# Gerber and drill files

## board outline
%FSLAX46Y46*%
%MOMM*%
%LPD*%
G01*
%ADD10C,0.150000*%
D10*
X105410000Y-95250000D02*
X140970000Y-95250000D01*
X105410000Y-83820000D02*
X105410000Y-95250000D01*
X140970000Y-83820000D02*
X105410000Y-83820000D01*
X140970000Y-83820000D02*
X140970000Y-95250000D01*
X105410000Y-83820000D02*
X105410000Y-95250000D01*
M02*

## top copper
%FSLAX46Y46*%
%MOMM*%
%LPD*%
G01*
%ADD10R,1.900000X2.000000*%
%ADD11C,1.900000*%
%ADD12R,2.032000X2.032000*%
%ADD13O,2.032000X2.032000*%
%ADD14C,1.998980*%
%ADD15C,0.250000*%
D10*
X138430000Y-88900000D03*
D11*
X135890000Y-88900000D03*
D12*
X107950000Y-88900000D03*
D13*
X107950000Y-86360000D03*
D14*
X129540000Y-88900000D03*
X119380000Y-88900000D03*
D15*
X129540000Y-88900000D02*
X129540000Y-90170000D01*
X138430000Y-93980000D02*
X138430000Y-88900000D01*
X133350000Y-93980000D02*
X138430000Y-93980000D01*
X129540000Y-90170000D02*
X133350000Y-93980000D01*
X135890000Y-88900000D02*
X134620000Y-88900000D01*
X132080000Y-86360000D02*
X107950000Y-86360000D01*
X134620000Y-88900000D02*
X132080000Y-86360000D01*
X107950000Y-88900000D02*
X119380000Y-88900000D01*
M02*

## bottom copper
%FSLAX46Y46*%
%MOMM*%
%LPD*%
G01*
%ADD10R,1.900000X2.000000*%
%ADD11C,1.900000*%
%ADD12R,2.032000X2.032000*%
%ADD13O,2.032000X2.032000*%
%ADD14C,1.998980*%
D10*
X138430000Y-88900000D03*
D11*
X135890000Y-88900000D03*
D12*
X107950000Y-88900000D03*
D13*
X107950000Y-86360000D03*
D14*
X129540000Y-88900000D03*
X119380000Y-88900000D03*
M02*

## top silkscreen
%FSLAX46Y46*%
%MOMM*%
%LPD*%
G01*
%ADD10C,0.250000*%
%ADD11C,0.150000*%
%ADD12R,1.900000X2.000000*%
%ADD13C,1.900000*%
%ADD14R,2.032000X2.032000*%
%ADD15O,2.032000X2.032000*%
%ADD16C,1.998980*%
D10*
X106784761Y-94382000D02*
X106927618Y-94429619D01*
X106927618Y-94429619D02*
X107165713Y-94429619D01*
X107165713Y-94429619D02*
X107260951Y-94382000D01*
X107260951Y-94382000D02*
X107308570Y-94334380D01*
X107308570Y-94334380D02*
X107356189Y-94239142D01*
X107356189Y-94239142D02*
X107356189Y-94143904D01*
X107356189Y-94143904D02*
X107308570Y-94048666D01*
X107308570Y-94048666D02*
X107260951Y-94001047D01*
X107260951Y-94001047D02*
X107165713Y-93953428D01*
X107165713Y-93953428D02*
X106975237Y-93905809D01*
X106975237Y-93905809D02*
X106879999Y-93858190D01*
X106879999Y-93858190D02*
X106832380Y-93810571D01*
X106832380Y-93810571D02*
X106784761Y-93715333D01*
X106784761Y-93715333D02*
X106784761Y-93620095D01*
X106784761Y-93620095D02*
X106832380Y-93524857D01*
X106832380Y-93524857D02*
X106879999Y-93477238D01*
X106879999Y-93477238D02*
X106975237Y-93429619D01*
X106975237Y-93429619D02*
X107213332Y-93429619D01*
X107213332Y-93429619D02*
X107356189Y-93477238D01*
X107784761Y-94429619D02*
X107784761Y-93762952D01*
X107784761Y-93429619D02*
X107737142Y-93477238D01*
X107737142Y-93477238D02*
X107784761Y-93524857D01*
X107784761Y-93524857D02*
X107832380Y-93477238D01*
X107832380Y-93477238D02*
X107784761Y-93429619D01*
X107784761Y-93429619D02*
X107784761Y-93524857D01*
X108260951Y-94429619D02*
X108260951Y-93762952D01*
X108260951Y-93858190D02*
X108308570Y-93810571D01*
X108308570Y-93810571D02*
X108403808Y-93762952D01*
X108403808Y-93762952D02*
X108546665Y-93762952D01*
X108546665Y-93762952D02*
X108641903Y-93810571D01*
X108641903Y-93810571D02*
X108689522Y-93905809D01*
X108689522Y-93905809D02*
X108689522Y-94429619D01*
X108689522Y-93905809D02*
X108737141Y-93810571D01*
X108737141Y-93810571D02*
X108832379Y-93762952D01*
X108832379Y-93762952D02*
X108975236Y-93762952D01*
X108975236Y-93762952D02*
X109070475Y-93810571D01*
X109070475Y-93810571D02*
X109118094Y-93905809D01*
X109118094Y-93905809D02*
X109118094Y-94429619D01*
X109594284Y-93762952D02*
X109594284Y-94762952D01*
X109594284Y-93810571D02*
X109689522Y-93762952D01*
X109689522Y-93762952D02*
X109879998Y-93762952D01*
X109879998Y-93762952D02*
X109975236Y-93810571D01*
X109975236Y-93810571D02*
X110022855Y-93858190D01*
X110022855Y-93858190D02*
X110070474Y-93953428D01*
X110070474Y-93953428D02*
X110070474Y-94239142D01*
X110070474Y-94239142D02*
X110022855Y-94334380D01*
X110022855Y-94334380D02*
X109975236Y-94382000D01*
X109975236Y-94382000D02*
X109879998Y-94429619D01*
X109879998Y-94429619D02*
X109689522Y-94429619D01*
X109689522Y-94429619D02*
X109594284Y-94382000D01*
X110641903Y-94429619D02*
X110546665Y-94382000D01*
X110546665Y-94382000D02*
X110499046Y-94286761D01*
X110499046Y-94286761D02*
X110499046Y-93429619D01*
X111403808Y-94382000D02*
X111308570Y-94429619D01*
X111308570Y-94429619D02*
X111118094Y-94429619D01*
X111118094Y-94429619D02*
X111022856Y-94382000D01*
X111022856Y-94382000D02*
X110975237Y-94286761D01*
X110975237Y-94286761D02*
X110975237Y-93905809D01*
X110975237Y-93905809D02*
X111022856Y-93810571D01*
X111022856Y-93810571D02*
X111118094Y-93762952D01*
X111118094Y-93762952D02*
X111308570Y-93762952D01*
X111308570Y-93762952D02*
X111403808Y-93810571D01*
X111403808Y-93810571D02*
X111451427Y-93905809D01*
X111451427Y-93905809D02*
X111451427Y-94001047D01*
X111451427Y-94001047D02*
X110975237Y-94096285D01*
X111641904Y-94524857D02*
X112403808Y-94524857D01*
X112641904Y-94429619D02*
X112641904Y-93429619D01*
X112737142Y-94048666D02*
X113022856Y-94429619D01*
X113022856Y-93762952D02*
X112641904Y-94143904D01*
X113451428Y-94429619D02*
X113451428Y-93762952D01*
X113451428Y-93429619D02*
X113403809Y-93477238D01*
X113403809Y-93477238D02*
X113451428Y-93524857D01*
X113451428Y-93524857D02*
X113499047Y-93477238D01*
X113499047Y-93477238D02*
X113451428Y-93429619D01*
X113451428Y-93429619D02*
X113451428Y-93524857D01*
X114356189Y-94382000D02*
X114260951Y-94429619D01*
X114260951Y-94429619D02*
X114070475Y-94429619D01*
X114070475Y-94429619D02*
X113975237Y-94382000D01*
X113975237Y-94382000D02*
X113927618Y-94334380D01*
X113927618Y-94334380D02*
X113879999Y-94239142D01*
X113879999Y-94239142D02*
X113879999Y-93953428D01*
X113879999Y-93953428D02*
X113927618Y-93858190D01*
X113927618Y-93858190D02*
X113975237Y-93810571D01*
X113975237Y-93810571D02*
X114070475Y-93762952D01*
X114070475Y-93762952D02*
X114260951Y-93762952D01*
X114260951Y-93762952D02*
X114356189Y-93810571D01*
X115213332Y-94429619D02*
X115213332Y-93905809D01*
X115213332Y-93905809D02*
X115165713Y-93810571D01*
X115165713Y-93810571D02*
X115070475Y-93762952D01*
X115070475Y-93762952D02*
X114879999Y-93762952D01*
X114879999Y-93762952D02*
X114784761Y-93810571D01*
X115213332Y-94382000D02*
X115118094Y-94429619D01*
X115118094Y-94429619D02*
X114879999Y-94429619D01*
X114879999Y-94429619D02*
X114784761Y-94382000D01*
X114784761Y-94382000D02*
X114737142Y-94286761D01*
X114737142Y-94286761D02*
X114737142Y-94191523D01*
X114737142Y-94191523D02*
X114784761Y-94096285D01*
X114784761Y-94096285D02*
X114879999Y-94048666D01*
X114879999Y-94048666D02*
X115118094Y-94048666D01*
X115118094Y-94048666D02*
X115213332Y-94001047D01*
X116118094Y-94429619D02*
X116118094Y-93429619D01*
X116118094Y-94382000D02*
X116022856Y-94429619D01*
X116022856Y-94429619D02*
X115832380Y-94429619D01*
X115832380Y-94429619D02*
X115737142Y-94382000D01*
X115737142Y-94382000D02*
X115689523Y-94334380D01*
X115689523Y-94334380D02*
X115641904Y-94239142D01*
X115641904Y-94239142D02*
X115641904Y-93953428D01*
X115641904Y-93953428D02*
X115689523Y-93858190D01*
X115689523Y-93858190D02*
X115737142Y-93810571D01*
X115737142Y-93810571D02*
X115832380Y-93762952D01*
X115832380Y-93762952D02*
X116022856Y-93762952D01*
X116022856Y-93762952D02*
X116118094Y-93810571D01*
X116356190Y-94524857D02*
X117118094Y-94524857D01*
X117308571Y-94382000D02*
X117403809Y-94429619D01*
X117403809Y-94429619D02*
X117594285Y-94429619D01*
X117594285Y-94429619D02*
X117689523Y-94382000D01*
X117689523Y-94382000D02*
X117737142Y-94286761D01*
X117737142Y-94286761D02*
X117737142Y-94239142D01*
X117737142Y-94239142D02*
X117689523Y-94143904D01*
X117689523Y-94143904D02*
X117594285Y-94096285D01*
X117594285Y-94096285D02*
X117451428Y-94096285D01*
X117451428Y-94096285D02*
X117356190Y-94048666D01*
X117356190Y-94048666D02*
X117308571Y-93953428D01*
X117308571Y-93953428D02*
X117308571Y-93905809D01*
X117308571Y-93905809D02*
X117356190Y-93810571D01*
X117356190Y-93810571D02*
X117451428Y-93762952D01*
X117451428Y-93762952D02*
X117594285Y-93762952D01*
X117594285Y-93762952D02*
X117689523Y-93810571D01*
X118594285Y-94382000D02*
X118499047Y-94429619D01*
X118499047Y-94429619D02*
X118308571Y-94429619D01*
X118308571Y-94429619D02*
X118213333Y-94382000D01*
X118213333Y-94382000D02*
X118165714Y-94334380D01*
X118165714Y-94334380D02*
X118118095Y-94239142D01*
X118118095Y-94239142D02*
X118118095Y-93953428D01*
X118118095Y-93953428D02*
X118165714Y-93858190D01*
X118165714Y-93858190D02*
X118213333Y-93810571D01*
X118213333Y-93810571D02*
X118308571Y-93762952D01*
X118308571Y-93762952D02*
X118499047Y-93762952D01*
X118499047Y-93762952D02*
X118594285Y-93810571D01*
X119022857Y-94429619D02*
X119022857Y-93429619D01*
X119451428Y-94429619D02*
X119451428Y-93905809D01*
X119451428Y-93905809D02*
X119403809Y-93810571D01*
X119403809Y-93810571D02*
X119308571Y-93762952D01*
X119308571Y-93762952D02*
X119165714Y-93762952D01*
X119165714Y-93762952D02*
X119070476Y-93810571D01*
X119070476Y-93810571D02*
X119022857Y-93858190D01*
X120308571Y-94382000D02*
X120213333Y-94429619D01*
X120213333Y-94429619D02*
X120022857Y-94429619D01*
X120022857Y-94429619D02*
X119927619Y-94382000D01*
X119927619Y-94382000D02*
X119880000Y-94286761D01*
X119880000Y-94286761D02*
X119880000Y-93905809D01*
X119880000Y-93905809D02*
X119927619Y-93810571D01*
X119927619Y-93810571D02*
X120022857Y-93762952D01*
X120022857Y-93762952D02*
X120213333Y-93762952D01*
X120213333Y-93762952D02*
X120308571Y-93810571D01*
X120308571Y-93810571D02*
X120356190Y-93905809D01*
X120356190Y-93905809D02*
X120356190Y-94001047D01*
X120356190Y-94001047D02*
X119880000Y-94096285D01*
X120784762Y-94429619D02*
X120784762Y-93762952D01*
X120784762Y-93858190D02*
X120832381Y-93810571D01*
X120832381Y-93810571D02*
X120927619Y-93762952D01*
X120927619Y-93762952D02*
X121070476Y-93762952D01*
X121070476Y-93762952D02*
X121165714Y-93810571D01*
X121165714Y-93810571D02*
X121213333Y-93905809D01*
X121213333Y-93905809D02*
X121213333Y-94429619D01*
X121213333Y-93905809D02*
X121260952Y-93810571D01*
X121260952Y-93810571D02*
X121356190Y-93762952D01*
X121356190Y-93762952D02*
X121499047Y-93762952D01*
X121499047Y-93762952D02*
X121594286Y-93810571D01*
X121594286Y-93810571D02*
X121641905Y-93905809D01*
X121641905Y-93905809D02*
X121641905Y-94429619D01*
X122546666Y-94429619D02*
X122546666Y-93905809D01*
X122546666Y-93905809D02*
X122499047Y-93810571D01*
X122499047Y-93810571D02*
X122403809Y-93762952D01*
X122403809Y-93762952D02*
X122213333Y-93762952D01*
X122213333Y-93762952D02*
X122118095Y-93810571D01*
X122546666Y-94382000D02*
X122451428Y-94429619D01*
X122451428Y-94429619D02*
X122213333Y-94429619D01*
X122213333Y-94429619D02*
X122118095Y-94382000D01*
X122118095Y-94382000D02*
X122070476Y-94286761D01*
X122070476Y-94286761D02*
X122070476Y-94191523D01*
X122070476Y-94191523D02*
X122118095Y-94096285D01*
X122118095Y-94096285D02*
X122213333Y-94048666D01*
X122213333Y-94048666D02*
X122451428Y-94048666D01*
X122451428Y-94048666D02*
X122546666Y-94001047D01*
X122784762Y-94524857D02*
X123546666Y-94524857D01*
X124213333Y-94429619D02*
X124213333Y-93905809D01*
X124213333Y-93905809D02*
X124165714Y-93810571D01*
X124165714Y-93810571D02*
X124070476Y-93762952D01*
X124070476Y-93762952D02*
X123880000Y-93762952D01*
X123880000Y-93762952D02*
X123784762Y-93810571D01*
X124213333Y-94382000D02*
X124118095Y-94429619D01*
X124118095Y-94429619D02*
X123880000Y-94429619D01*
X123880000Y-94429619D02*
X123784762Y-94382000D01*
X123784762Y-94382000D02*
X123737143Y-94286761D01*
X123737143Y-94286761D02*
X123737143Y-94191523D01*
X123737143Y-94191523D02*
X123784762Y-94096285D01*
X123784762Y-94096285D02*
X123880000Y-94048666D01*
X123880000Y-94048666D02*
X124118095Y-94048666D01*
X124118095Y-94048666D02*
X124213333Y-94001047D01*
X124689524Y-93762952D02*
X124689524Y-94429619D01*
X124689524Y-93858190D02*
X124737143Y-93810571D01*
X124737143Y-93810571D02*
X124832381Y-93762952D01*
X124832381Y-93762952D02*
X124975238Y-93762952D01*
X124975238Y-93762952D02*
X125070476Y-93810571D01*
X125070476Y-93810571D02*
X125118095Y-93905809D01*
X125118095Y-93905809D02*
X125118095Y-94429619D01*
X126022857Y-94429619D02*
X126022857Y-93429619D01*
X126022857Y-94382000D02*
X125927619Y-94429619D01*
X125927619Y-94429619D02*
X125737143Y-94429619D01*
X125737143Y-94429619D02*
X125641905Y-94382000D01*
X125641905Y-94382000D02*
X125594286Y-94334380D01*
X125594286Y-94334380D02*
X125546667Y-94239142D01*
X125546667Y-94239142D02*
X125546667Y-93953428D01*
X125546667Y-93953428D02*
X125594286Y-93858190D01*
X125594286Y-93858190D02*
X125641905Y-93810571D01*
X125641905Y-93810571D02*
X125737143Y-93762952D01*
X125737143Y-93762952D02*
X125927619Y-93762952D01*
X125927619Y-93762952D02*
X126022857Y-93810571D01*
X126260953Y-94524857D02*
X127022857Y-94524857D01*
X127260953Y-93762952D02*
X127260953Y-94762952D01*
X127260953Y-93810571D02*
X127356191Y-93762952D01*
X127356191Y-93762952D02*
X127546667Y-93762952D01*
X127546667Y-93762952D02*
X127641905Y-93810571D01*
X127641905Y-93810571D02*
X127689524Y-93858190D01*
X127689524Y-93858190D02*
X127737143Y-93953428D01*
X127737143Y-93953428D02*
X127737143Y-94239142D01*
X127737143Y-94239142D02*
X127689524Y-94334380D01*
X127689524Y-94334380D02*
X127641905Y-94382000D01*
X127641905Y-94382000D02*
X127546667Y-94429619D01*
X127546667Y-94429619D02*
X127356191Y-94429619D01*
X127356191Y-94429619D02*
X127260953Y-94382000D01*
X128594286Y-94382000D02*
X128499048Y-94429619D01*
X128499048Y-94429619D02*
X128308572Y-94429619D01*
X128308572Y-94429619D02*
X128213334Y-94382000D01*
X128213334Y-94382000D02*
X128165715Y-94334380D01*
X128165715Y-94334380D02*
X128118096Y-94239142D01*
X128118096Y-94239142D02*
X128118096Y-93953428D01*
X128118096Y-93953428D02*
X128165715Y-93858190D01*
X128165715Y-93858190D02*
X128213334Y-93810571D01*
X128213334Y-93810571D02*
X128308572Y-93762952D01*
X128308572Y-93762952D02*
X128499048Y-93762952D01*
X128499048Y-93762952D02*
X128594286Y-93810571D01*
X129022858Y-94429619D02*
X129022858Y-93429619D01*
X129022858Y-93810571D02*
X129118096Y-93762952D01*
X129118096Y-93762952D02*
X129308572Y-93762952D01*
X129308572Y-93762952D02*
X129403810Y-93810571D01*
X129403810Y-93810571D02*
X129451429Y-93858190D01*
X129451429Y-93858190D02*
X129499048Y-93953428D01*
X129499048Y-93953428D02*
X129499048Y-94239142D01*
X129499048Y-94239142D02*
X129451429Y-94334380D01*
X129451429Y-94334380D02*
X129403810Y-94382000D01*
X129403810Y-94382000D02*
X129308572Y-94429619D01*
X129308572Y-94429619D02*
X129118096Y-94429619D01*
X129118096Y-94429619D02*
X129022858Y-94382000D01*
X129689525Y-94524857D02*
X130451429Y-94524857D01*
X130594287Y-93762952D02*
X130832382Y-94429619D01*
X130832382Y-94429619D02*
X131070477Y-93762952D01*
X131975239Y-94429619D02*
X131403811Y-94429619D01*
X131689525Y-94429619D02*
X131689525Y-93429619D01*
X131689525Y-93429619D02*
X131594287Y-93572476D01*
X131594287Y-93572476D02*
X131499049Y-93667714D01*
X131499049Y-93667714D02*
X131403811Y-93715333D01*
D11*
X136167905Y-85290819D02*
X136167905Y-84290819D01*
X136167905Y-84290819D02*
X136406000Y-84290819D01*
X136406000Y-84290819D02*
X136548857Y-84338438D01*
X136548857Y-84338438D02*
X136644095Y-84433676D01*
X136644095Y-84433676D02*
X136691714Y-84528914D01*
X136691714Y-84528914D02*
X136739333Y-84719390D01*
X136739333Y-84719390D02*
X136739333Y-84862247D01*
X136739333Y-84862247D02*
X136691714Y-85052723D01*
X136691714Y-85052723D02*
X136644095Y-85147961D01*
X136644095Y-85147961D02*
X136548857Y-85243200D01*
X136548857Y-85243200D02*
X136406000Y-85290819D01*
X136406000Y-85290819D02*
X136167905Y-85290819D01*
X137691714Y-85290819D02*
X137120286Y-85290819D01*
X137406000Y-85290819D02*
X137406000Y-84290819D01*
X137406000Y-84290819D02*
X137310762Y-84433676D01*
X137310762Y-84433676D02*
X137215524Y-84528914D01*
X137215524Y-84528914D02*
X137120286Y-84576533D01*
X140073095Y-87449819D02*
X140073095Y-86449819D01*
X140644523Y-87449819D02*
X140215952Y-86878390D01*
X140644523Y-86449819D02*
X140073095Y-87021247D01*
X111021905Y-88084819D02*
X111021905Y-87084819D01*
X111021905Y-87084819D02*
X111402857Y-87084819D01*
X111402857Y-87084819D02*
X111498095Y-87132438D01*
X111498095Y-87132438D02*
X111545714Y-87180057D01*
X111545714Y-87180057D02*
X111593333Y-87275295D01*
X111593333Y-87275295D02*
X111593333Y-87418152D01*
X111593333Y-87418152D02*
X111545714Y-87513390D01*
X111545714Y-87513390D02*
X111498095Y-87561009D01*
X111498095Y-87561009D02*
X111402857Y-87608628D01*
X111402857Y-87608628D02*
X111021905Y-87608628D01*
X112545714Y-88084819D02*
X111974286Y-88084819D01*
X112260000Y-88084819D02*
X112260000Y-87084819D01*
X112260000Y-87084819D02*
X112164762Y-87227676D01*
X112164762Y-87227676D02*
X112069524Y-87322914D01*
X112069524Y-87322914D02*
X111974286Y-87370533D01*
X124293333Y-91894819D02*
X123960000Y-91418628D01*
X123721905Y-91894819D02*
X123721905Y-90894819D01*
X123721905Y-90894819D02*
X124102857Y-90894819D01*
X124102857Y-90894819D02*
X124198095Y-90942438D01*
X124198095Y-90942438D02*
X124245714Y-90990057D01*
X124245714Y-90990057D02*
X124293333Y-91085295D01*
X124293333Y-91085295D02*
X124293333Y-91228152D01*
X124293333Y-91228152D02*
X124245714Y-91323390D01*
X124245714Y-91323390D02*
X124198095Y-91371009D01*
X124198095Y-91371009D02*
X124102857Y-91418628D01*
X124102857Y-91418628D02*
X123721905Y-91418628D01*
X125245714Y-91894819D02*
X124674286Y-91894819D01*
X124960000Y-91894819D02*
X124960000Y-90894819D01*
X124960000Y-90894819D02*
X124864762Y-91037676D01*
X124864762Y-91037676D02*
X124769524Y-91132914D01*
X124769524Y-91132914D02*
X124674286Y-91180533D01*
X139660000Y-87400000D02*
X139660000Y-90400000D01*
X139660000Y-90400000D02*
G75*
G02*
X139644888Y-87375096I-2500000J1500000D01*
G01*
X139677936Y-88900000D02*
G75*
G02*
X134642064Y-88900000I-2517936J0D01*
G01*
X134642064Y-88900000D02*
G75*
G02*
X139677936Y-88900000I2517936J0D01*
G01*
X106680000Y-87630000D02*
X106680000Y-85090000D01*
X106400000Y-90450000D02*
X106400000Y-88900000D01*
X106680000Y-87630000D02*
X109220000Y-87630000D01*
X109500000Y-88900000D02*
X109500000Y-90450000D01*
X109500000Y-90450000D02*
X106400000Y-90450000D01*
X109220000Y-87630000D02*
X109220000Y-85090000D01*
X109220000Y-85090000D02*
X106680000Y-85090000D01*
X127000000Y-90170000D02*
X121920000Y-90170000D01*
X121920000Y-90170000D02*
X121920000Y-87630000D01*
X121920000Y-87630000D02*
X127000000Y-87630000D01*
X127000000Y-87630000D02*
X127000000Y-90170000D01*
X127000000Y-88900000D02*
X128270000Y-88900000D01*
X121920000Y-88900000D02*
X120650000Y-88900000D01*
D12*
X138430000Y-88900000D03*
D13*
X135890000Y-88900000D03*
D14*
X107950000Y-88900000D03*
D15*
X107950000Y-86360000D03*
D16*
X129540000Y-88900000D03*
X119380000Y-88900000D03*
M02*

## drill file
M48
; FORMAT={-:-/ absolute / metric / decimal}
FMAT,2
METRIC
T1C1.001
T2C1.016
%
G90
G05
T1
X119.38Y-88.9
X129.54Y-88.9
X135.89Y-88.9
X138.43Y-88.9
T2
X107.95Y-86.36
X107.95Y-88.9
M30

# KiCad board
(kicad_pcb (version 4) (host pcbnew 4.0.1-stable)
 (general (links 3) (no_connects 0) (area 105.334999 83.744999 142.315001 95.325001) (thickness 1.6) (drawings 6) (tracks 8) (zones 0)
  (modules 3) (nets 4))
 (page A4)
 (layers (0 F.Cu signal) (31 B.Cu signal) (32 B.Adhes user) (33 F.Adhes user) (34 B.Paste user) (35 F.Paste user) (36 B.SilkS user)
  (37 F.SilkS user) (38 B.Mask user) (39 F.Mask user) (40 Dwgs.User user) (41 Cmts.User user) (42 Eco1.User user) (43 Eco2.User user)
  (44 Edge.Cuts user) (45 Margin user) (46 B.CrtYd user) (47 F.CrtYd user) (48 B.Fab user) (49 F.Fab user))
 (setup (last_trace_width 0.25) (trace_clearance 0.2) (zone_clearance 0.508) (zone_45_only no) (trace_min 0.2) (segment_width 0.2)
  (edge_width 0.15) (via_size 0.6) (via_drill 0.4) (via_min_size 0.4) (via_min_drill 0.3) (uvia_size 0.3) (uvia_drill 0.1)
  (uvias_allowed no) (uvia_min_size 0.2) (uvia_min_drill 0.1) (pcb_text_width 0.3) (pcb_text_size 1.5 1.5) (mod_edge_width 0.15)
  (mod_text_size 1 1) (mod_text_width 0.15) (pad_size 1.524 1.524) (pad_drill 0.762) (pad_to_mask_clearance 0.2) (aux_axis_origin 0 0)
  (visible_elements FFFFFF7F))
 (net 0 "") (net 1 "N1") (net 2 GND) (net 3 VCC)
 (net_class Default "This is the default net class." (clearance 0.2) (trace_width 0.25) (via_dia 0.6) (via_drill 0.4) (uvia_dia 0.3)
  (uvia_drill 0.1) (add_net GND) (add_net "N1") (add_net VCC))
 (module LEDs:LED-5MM (layer F.Cu) (at 138.43 88.9 180)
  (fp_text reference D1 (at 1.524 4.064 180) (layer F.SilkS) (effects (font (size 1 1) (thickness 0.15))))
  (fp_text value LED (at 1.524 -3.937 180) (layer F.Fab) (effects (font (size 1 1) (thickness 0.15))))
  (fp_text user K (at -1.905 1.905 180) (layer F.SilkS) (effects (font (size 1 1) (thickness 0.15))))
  (fp_line (start -1.23 1.5) (end -1.23 -1.5) (layer F.SilkS) (width 0.15))
  (fp_arc (start 1.27 0) (end -1.23 -1.5) (angle 297.5) (layer F.SilkS) (width 0.15))
  (fp_circle (center 1.27 0) (end 0.97 -2.5) (layer F.SilkS) (width 0.15))
  (pad 1 thru_hole rect (at 0 0 270) (size 2 1.9) (drill 1.00076) (layers *.Cu *.Mask F.SilkS) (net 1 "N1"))
  (pad 2 thru_hole circle (at 2.54 0 180) (size 1.9 1.9) (drill 1.00076) (layers *.Cu *.Mask F.SilkS) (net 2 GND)))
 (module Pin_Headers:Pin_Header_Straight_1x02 (layer F.Cu) (at 107.95 88.9 180)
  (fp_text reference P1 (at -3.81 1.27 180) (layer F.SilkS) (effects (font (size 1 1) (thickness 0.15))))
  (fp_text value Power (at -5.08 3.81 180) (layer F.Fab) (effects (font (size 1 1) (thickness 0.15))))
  (fp_line (start 1.27 1.27) (end 1.27 3.81) (layer F.SilkS) (width 0.15))
  (fp_line (start 1.55 -1.55) (end 1.55 0) (layer F.SilkS) (width 0.15))
  (fp_line (start 1.27 1.27) (end -1.27 1.27) (layer F.SilkS) (width 0.15))
  (fp_line (start -1.55 0) (end -1.55 -1.55) (layer F.SilkS) (width 0.15))
  (fp_line (start -1.55 -1.55) (end 1.55 -1.55) (layer F.SilkS) (width 0.15))
  (fp_line (start -1.27 1.27) (end -1.27 3.81) (layer F.SilkS) (width 0.15))
  (fp_line (start -1.27 3.81) (end 1.27 3.81) (layer F.SilkS) (width 0.15))
  (pad 1 thru_hole rect (at 0 0 180) (size 2.032 2.032) (drill 1.016) (layers *.Cu *.Mask F.SilkS) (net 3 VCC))
  (pad 2 thru_hole oval (at 0 2.54 180) (size 2.032 2.032) (drill 1.016) (layers *.Cu *.Mask F.SilkS) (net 2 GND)))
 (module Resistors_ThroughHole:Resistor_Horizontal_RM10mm (layer F.Cu) (at 124.46 88.9 180)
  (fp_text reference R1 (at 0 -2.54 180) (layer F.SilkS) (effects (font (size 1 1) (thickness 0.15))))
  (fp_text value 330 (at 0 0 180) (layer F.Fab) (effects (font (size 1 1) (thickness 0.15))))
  (fp_line (start -2.54 -1.27) (end 2.54 -1.27) (layer F.SilkS) (width 0.15))
  (fp_line (start 2.54 -1.27) (end 2.54 1.27) (layer F.SilkS) (width 0.15))
  (fp_line (start 2.54 1.27) (end -2.54 1.27) (layer F.SilkS) (width 0.15))
  (fp_line (start -2.54 1.27) (end -2.54 -1.27) (layer F.SilkS) (width 0.15))
  (fp_line (start -2.54 0) (end -3.81 0) (layer F.SilkS) (width 0.15))
  (fp_line (start 2.54 0) (end 3.81 0) (layer F.SilkS) (width 0.15))
  (pad 1 thru_hole circle (at -5.08 0 180) (size 1.99898 1.99898) (drill 1.00076) (layers *.Cu *.SilkS *.Mask) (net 1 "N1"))
  (pad 2 thru_hole circle (at 5.08 0 180) (size 1.99898 1.99898) (drill 1.00076) (layers *.Cu *.SilkS *.Mask) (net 3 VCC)))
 (gr_line (start 105.41 95.25) (end 140.97 95.25) (angle 90) (layer Edge.Cuts) (width 0.15))
 (gr_line (start 105.41 83.82) (end 105.41 95.25) (angle 90) (layer Edge.Cuts) (width 0.15))
 (gr_line (start 140.97 83.82) (end 105.41 83.82) (angle 90) (layer Edge.Cuts) (width 0.15))
 (gr_line (start 140.97 83.82) (end 140.97 95.25) (angle 90) (layer Edge.Cuts) (width 0.15))
 (gr_line (start 105.41 83.82) (end 105.41 95.25) (angle 90) (layer Edge.Cuts) (width 0.15))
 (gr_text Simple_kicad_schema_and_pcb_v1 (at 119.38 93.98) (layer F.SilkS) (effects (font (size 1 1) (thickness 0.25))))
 (segment (start 129.54 88.9) (end 129.54 90.17) (width 0.25) (layer F.Cu) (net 1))
 (segment (start 138.43 93.98) (end 138.43 88.9) (width 0.25) (layer F.Cu) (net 1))
 (segment (start 133.35 93.98) (end 138.43 93.98) (width 0.25) (layer F.Cu) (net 1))
 (segment (start 129.54 90.17) (end 133.35 93.98) (width 0.25) (layer F.Cu) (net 1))
 (segment (start 135.89 88.9) (end 134.62 88.9) (width 0.25) (layer F.Cu) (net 2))
 (segment (start 132.08 86.36) (end 107.95 86.36) (width 0.25) (layer F.Cu) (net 2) (status 20))
 (segment (start 134.62 88.9) (end 132.08 86.36) (width 0.25) (layer F.Cu) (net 2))
 (segment (start 107.95 88.9) (end 119.38 88.9) (width 0.25) (layer F.Cu) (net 3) (status 10)))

